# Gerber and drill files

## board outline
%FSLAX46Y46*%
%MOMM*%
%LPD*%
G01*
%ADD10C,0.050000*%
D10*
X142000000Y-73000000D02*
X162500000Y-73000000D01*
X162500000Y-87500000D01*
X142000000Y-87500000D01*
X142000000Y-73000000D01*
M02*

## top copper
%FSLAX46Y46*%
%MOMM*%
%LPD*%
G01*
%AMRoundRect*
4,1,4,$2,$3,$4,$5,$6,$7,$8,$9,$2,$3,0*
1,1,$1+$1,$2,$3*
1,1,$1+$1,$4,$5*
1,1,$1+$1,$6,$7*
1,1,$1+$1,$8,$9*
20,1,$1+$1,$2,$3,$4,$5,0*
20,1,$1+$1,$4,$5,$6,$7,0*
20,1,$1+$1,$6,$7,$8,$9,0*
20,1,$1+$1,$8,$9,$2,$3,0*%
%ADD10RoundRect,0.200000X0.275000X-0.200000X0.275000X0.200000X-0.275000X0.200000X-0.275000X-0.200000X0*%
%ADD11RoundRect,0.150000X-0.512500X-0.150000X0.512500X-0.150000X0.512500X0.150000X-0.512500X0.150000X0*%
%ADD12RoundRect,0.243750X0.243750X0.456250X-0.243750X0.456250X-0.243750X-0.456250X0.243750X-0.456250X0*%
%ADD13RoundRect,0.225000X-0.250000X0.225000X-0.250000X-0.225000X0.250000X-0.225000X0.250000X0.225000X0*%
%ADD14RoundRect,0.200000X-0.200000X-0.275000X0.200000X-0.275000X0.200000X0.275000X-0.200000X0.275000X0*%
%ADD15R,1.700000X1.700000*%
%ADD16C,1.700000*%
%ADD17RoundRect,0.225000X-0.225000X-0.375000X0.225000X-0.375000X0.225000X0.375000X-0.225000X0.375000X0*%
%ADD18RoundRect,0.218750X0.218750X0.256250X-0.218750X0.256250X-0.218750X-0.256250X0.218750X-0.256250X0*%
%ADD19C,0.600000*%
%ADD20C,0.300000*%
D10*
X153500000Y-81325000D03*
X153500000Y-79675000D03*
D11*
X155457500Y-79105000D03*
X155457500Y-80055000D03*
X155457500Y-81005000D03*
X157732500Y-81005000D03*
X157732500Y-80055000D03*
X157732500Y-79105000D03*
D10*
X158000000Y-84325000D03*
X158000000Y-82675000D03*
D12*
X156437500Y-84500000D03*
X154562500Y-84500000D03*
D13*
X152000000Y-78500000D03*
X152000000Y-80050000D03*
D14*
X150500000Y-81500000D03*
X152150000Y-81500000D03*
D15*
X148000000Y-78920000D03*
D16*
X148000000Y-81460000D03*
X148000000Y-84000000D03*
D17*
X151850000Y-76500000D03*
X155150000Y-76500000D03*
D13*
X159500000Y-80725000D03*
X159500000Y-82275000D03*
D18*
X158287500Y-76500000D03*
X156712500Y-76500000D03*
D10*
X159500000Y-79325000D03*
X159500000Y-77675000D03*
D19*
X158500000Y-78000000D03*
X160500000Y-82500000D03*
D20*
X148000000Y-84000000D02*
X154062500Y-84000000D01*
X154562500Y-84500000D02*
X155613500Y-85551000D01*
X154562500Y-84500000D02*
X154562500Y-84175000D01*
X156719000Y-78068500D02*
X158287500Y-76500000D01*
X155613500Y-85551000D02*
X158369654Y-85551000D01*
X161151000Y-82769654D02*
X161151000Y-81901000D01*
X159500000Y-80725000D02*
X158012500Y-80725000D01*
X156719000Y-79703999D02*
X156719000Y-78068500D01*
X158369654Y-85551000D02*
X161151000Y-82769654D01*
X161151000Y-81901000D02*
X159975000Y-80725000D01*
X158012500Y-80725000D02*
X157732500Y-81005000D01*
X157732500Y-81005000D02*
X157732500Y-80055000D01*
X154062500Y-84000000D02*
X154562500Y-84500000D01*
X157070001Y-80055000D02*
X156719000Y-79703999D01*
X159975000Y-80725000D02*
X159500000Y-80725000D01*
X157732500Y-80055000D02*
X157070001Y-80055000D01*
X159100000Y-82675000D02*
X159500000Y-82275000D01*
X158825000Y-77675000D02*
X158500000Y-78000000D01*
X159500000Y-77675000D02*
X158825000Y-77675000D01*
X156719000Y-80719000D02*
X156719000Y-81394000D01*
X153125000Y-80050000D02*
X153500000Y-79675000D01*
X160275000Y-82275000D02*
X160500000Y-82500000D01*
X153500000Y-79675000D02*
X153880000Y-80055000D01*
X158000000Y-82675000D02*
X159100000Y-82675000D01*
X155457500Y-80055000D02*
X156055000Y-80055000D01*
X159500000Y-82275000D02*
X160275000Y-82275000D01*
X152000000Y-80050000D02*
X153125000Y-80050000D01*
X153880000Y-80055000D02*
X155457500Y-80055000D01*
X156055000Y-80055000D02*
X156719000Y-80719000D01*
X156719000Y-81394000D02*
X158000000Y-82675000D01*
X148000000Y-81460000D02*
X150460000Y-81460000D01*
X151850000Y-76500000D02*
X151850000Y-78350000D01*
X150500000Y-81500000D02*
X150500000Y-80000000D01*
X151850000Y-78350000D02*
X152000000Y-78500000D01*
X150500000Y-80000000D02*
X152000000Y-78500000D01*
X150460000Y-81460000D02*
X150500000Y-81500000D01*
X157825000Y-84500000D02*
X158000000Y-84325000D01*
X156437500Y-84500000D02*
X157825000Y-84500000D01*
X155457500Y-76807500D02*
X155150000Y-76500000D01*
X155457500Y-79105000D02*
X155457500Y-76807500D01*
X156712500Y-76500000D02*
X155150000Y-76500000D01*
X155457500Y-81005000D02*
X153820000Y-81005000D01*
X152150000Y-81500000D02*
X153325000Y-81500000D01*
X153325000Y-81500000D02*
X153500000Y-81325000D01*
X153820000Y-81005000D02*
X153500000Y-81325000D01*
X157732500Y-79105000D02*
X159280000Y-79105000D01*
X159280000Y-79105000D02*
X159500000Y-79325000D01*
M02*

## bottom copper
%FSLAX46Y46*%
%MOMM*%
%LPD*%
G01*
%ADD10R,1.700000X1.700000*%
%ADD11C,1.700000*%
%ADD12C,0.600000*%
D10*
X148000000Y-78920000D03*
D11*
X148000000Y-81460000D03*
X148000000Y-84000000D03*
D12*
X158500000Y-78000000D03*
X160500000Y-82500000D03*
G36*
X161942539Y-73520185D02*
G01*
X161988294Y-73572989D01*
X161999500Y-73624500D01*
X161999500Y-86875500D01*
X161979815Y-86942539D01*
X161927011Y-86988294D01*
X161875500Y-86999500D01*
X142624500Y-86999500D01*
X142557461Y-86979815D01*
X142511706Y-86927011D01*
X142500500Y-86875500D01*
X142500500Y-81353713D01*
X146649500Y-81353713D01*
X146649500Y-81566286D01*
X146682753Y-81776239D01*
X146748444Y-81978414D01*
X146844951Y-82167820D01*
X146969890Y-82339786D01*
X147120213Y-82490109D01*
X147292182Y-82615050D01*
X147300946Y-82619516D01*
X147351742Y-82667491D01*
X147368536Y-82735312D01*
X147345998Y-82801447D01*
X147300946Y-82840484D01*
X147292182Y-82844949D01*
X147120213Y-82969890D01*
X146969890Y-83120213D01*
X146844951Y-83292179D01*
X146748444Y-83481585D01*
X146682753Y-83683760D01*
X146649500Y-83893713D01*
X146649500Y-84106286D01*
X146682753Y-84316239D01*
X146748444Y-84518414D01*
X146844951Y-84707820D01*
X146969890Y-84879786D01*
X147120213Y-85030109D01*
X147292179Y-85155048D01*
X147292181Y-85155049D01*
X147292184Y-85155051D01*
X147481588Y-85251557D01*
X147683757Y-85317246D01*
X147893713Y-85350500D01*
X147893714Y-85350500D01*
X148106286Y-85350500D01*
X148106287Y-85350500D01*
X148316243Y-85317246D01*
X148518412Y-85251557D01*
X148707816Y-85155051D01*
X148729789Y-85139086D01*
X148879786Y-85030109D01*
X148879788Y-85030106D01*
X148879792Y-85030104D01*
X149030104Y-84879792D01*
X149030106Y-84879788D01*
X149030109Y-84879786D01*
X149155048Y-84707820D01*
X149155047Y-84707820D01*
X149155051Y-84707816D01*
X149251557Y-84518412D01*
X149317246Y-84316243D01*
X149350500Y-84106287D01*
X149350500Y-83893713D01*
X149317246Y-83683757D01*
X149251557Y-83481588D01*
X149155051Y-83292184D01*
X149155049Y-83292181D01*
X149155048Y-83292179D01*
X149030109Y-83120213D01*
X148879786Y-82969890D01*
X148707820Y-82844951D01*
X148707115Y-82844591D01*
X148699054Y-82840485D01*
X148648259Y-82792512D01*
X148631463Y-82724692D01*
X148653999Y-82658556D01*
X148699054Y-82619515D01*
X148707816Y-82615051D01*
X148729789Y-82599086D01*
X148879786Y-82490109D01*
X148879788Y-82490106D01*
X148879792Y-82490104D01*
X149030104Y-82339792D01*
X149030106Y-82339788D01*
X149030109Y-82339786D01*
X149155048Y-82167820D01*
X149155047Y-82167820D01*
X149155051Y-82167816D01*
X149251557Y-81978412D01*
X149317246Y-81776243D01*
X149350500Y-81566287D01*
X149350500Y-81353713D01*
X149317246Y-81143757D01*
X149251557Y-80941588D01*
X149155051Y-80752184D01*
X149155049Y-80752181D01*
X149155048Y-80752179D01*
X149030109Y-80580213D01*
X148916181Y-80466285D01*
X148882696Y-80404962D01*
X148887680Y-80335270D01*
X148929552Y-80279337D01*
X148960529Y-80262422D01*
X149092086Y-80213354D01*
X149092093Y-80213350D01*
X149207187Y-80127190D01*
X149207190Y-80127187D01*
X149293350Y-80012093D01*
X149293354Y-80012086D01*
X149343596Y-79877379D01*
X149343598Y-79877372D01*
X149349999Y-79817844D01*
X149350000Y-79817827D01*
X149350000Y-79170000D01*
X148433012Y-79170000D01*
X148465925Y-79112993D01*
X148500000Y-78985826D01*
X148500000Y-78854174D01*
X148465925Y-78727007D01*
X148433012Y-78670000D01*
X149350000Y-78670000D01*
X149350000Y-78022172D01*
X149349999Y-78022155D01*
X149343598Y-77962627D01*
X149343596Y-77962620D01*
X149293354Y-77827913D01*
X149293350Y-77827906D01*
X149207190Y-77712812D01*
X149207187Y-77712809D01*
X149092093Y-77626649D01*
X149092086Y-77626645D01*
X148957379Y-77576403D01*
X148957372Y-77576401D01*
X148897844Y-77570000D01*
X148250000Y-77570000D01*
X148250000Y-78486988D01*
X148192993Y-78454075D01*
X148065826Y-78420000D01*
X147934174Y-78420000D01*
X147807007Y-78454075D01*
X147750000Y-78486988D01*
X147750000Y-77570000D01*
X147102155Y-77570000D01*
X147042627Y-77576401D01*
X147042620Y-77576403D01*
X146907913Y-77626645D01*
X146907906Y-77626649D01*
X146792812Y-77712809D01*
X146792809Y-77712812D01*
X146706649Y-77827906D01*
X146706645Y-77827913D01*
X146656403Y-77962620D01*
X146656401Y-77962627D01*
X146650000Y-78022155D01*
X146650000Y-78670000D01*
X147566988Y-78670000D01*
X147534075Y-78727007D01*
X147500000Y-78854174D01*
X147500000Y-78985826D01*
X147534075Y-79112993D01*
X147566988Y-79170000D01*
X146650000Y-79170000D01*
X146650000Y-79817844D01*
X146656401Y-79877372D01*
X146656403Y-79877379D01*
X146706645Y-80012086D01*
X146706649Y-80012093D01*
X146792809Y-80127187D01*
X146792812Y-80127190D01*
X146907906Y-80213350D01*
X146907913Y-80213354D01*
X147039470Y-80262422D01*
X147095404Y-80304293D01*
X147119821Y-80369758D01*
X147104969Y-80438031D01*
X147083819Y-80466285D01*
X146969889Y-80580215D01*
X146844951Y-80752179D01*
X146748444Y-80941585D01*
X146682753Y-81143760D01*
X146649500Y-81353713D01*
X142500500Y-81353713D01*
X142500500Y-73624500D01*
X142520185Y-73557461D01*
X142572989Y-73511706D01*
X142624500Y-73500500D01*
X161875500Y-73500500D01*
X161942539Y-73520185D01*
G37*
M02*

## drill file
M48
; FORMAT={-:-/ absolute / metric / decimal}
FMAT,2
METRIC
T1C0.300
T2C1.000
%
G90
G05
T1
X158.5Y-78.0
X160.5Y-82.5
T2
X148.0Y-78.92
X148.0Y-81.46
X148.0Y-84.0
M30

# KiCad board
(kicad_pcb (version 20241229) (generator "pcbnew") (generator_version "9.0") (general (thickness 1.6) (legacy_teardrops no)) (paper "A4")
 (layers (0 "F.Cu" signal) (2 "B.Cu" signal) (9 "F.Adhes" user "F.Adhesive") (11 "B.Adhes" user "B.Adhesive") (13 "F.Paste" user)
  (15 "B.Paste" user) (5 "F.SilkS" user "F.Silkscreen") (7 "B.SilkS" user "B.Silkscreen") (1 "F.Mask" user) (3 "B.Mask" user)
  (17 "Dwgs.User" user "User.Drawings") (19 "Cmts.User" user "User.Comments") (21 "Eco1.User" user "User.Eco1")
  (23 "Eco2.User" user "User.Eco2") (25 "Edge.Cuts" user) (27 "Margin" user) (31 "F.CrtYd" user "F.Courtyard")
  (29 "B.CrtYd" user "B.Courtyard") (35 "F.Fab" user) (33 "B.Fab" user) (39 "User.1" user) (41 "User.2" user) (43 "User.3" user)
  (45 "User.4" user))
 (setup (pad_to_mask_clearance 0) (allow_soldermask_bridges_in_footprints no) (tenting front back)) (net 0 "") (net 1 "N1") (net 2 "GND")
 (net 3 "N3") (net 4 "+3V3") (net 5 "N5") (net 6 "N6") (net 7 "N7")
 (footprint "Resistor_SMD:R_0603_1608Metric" (layer "F.Cu") (at 153.5 80.5 90)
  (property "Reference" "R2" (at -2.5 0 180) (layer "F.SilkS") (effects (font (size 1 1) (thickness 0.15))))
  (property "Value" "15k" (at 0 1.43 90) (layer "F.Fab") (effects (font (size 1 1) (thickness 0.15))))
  (pad "1" smd roundrect (at -0.825 0 90) (size 0.8 0.95) (layers "F.Cu" "F.Mask" "F.Paste") (roundrect_rratio 0.25) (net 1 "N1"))
  (pad "2" smd roundrect (at 0.825 0 90) (size 0.8 0.95) (layers "F.Cu" "F.Mask" "F.Paste") (roundrect_rratio 0.25) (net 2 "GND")))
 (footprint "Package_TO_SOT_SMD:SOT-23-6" (layer "F.Cu") (at 156.595 80.055)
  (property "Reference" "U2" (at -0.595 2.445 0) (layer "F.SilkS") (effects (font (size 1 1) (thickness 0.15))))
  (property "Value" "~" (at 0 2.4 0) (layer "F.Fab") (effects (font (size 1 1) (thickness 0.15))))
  (pad "1" smd roundrect (at -1.1375 -0.95) (size 1.325 0.6) (layers "F.Cu" "F.Mask" "F.Paste") (roundrect_rratio 0.25) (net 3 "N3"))
  (pad "2" smd roundrect (at -1.1375 0) (size 1.325 0.6) (layers "F.Cu" "F.Mask" "F.Paste") (roundrect_rratio 0.25) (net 2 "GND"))
  (pad "3" smd roundrect (at -1.1375 0.95) (size 1.325 0.6) (layers "F.Cu" "F.Mask" "F.Paste") (roundrect_rratio 0.25) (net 1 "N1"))
  (pad "4" smd roundrect (at 1.1375 0.95) (size 1.325 0.6) (layers "F.Cu" "F.Mask" "F.Paste") (roundrect_rratio 0.25) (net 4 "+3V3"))
  (pad "5" smd roundrect (at 1.1375 0) (size 1.325 0.6) (layers "F.Cu" "F.Mask" "F.Paste") (roundrect_rratio 0.25) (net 4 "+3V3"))
  (pad "6" smd roundrect (at 1.1375 -0.95) (size 1.325 0.6) (layers "F.Cu" "F.Mask" "F.Paste") (roundrect_rratio 0.25) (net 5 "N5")))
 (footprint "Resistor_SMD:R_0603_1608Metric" (layer "F.Cu") (at 158 83.5 90)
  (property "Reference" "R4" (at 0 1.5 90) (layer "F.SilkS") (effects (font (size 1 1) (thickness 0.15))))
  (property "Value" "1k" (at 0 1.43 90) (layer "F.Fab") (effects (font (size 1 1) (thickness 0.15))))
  (pad "1" smd roundrect (at -0.825 0 90) (size 0.8 0.95) (layers "F.Cu" "F.Mask" "F.Paste") (roundrect_rratio 0.25) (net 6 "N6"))
  (pad "2" smd roundrect (at 0.825 0 90) (size 0.8 0.95) (layers "F.Cu" "F.Mask" "F.Paste") (roundrect_rratio 0.25) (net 2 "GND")))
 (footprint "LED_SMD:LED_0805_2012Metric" (layer "F.Cu") (at 155.5 84.5 180)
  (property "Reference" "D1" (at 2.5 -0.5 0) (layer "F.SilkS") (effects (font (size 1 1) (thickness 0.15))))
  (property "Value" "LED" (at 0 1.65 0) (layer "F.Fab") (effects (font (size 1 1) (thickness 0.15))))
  (pad "1" smd roundrect (at -0.9375 0 180) (size 0.975 1.4) (layers "F.Cu" "F.Mask" "F.Paste") (roundrect_rratio 0.25) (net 6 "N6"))
  (pad "2" smd roundrect (at 0.9375 0 180) (size 0.975 1.4) (layers "F.Cu" "F.Mask" "F.Paste") (roundrect_rratio 0.25) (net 4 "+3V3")))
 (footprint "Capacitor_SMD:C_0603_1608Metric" (layer "F.Cu") (at 152 79.275 -90)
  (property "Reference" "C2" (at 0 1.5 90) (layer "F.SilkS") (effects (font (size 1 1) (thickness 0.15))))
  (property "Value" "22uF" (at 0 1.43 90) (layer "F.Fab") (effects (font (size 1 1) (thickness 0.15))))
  (pad "1" smd roundrect (at -0.775 0 270) (size 0.9 0.95) (layers "F.Cu" "F.Mask" "F.Paste") (roundrect_rratio 0.25) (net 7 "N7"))
  (pad "2" smd roundrect (at 0.775 0 270) (size 0.9 0.95) (layers "F.Cu" "F.Mask" "F.Paste") (roundrect_rratio 0.25) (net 2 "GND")))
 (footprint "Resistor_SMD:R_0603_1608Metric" (layer "F.Cu") (at 151.325 81.5)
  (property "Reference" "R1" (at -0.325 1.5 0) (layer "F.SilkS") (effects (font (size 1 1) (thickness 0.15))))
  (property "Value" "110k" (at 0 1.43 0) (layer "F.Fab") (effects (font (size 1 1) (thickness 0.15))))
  (pad "1" smd roundrect (at -0.825 0) (size 0.8 0.95) (layers "F.Cu" "F.Mask" "F.Paste") (roundrect_rratio 0.25) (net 7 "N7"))
  (pad "2" smd roundrect (at 0.825 0) (size 0.8 0.95) (layers "F.Cu" "F.Mask" "F.Paste") (roundrect_rratio 0.25) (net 1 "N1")))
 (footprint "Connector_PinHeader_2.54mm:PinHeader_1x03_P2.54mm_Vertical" (layer "F.Cu") (at 148 78.92)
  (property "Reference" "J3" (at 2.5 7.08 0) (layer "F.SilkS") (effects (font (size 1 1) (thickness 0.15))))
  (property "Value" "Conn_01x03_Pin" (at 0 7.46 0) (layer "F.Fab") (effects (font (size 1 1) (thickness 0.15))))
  (pad "1" thru_hole rect (at 0 0) (size 1.7 1.7) (drill 1) (layers "*.Cu" "*.Mask") (remove_unused_layers no) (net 2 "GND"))
  (pad "2" thru_hole circle (at 0 2.54) (size 1.7 1.7) (drill 1) (layers "*.Cu" "*.Mask") (remove_unused_layers no) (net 7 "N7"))
  (pad "3" thru_hole circle (at 0 5.08) (size 1.7 1.7) (drill 1) (layers "*.Cu" "*.Mask") (remove_unused_layers no) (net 4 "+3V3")))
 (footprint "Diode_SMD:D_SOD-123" (layer "F.Cu") (at 153.5 76.5)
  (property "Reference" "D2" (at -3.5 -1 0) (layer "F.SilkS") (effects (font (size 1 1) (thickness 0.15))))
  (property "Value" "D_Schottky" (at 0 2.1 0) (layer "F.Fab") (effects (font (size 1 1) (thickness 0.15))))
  (pad "1" smd roundrect (at -1.65 0) (size 0.9 1.2) (layers "F.Cu" "F.Mask" "F.Paste") (roundrect_rratio 0.25) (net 7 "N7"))
  (pad "2" smd roundrect (at 1.65 0) (size 0.9 1.2) (layers "F.Cu" "F.Mask" "F.Paste") (roundrect_rratio 0.25) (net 3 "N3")))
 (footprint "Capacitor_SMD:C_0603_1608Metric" (layer "F.Cu") (at 159.5 81.5 -90)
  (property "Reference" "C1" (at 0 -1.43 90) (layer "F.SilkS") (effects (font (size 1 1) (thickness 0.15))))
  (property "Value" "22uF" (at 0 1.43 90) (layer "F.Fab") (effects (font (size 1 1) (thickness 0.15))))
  (pad "1" smd roundrect (at -0.775 0 270) (size 0.9 0.95) (layers "F.Cu" "F.Mask" "F.Paste") (roundrect_rratio 0.25) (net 4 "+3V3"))
  (pad "2" smd roundrect (at 0.775 0 270) (size 0.9 0.95) (layers "F.Cu" "F.Mask" "F.Paste") (roundrect_rratio 0.25) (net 2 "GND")))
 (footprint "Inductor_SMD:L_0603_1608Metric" (layer "F.Cu") (at 157.5 76.5 180)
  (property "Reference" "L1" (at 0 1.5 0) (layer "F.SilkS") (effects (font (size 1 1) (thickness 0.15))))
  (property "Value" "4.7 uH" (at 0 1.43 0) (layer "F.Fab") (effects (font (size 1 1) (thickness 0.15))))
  (pad "1" smd roundrect (at -0.7875 0 180) (size 0.875 0.95) (layers "F.Cu" "F.Mask" "F.Paste") (roundrect_rratio 0.25) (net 4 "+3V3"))
  (pad "2" smd roundrect (at 0.7875 0 180) (size 0.875 0.95) (layers "F.Cu" "F.Mask" "F.Paste") (roundrect_rratio 0.25) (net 3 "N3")))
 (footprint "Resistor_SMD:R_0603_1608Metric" (layer "F.Cu") (at 159.5 78.5 90)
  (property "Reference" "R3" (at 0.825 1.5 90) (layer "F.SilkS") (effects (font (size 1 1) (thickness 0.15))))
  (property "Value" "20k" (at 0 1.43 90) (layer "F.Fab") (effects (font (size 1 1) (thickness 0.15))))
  (pad "1" smd roundrect (at -0.825 0 90) (size 0.8 0.95) (layers "F.Cu" "F.Mask" "F.Paste") (roundrect_rratio 0.25) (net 5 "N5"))
  (pad "2" smd roundrect (at 0.825 0 90) (size 0.8 0.95) (layers "F.Cu" "F.Mask" "F.Paste") (roundrect_rratio 0.25) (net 2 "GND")))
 (gr_rect (start 142 73) (end 162.5 87.5) (stroke (width 0.05) (type default)) (fill no) (layer "Edge.Cuts"))
 (segment (start 148 84) (end 154.0625 84) (width 0.3) (layer "F.Cu") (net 4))
 (segment (start 154.5625 84.5) (end 155.6135 85.551) (width 0.3) (layer "F.Cu") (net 4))
 (segment (start 154.5625 84.5) (end 154.5625 84.175) (width 0.3) (layer "F.Cu") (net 4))
 (segment (start 156.719 78.0685) (end 158.2875 76.5) (width 0.3) (layer "F.Cu") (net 4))
 (segment (start 155.6135 85.551) (end 158.369654 85.551) (width 0.3) (layer "F.Cu") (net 4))
 (segment (start 161.151 82.769654) (end 161.151 81.901) (width 0.3) (layer "F.Cu") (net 4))
 (segment (start 159.5 80.725) (end 158.0125 80.725) (width 0.3) (layer "F.Cu") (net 4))
 (segment (start 156.719 79.703999) (end 156.719 78.0685) (width 0.3) (layer "F.Cu") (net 4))
 (segment (start 158.369654 85.551) (end 161.151 82.769654) (width 0.3) (layer "F.Cu") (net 4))
 (segment (start 161.151 81.901) (end 159.975 80.725) (width 0.3) (layer "F.Cu") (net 4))
 (segment (start 158.0125 80.725) (end 157.7325 81.005) (width 0.3) (layer "F.Cu") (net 4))
 (segment (start 157.7325 81.005) (end 157.7325 80.055) (width 0.3) (layer "F.Cu") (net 4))
 (segment (start 154.0625 84) (end 154.5625 84.5) (width 0.3) (layer "F.Cu") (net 4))
 (segment (start 157.070001 80.055) (end 156.719 79.703999) (width 0.3) (layer "F.Cu") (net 4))
 (segment (start 159.975 80.725) (end 159.5 80.725) (width 0.3) (layer "F.Cu") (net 4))
 (segment (start 157.7325 80.055) (end 157.070001 80.055) (width 0.3) (layer "F.Cu") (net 4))
 (segment (start 159.1 82.675) (end 159.5 82.275) (width 0.3) (layer "F.Cu") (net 2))
 (segment (start 158.825 77.675) (end 158.5 78) (width 0.3) (layer "F.Cu") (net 2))
 (segment (start 159.5 77.675) (end 158.825 77.675) (width 0.3) (layer "F.Cu") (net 2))
 (segment (start 156.719 80.719) (end 156.719 81.394) (width 0.3) (layer "F.Cu") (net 2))
 (segment (start 153.125 80.05) (end 153.5 79.675) (width 0.3) (layer "F.Cu") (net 2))
 (segment (start 160.275 82.275) (end 160.5 82.5) (width 0.3) (layer "F.Cu") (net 2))
 (segment (start 153.5 79.675) (end 153.88 80.055) (width 0.3) (layer "F.Cu") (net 2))
 (segment (start 158 82.675) (end 159.1 82.675) (width 0.3) (layer "F.Cu") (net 2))
 (segment (start 155.4575 80.055) (end 156.055 80.055) (width 0.3) (layer "F.Cu") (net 2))
 (segment (start 159.5 82.275) (end 160.275 82.275) (width 0.3) (layer "F.Cu") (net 2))
 (segment (start 152 80.05) (end 153.125 80.05) (width 0.3) (layer "F.Cu") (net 2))
 (segment (start 153.88 80.055) (end 155.4575 80.055) (width 0.3) (layer "F.Cu") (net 2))
 (segment (start 156.055 80.055) (end 156.719 80.719) (width 0.3) (layer "F.Cu") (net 2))
 (segment (start 156.719 81.394) (end 158 82.675) (width 0.3) (layer "F.Cu") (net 2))
 (via (at 158.5 78) (size 0.6) (drill 0.3) (layers "F.Cu" "B.Cu") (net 2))
 (via (at 160.5 82.5) (size 0.6) (drill 0.3) (layers "F.Cu" "B.Cu") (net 2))
 (segment (start 148 81.46) (end 150.46 81.46) (width 0.3) (layer "F.Cu") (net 7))
 (segment (start 151.85 76.5) (end 151.85 78.35) (width 0.3) (layer "F.Cu") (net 7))
 (segment (start 150.5 81.5) (end 150.5 80) (width 0.3) (layer "F.Cu") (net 7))
 (segment (start 151.85 78.35) (end 152 78.5) (width 0.3) (layer "F.Cu") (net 7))
 (segment (start 150.5 80) (end 152 78.5) (width 0.3) (layer "F.Cu") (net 7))
 (segment (start 150.46 81.46) (end 150.5 81.5) (width 0.3) (layer "F.Cu") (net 7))
 (segment (start 157.825 84.5) (end 158 84.325) (width 0.3) (layer "F.Cu") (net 6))
 (segment (start 156.4375 84.5) (end 157.825 84.5) (width 0.3) (layer "F.Cu") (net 6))
 (segment (start 155.4575 76.8075) (end 155.15 76.5) (width 0.3) (layer "F.Cu") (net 3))
 (segment (start 155.4575 79.105) (end 155.4575 76.8075) (width 0.3) (layer "F.Cu") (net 3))
 (segment (start 156.7125 76.5) (end 155.15 76.5) (width 0.3) (layer "F.Cu") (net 3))
 (segment (start 155.4575 81.005) (end 153.82 81.005) (width 0.3) (layer "F.Cu") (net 1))
 (segment (start 152.15 81.5) (end 153.325 81.5) (width 0.3) (layer "F.Cu") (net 1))
 (segment (start 153.325 81.5) (end 153.5 81.325) (width 0.3) (layer "F.Cu") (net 1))
 (segment (start 153.82 81.005) (end 153.5 81.325) (width 0.3) (layer "F.Cu") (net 1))
 (segment (start 157.7325 79.105) (end 159.28 79.105) (width 0.3) (layer "F.Cu") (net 5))
 (segment (start 159.28 79.105) (end 159.5 79.325) (width 0.3) (layer "F.Cu") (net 5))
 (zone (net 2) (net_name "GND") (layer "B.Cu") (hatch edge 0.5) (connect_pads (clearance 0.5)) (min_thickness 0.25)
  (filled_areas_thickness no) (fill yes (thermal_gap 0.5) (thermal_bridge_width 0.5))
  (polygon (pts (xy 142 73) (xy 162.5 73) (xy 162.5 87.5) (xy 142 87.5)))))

